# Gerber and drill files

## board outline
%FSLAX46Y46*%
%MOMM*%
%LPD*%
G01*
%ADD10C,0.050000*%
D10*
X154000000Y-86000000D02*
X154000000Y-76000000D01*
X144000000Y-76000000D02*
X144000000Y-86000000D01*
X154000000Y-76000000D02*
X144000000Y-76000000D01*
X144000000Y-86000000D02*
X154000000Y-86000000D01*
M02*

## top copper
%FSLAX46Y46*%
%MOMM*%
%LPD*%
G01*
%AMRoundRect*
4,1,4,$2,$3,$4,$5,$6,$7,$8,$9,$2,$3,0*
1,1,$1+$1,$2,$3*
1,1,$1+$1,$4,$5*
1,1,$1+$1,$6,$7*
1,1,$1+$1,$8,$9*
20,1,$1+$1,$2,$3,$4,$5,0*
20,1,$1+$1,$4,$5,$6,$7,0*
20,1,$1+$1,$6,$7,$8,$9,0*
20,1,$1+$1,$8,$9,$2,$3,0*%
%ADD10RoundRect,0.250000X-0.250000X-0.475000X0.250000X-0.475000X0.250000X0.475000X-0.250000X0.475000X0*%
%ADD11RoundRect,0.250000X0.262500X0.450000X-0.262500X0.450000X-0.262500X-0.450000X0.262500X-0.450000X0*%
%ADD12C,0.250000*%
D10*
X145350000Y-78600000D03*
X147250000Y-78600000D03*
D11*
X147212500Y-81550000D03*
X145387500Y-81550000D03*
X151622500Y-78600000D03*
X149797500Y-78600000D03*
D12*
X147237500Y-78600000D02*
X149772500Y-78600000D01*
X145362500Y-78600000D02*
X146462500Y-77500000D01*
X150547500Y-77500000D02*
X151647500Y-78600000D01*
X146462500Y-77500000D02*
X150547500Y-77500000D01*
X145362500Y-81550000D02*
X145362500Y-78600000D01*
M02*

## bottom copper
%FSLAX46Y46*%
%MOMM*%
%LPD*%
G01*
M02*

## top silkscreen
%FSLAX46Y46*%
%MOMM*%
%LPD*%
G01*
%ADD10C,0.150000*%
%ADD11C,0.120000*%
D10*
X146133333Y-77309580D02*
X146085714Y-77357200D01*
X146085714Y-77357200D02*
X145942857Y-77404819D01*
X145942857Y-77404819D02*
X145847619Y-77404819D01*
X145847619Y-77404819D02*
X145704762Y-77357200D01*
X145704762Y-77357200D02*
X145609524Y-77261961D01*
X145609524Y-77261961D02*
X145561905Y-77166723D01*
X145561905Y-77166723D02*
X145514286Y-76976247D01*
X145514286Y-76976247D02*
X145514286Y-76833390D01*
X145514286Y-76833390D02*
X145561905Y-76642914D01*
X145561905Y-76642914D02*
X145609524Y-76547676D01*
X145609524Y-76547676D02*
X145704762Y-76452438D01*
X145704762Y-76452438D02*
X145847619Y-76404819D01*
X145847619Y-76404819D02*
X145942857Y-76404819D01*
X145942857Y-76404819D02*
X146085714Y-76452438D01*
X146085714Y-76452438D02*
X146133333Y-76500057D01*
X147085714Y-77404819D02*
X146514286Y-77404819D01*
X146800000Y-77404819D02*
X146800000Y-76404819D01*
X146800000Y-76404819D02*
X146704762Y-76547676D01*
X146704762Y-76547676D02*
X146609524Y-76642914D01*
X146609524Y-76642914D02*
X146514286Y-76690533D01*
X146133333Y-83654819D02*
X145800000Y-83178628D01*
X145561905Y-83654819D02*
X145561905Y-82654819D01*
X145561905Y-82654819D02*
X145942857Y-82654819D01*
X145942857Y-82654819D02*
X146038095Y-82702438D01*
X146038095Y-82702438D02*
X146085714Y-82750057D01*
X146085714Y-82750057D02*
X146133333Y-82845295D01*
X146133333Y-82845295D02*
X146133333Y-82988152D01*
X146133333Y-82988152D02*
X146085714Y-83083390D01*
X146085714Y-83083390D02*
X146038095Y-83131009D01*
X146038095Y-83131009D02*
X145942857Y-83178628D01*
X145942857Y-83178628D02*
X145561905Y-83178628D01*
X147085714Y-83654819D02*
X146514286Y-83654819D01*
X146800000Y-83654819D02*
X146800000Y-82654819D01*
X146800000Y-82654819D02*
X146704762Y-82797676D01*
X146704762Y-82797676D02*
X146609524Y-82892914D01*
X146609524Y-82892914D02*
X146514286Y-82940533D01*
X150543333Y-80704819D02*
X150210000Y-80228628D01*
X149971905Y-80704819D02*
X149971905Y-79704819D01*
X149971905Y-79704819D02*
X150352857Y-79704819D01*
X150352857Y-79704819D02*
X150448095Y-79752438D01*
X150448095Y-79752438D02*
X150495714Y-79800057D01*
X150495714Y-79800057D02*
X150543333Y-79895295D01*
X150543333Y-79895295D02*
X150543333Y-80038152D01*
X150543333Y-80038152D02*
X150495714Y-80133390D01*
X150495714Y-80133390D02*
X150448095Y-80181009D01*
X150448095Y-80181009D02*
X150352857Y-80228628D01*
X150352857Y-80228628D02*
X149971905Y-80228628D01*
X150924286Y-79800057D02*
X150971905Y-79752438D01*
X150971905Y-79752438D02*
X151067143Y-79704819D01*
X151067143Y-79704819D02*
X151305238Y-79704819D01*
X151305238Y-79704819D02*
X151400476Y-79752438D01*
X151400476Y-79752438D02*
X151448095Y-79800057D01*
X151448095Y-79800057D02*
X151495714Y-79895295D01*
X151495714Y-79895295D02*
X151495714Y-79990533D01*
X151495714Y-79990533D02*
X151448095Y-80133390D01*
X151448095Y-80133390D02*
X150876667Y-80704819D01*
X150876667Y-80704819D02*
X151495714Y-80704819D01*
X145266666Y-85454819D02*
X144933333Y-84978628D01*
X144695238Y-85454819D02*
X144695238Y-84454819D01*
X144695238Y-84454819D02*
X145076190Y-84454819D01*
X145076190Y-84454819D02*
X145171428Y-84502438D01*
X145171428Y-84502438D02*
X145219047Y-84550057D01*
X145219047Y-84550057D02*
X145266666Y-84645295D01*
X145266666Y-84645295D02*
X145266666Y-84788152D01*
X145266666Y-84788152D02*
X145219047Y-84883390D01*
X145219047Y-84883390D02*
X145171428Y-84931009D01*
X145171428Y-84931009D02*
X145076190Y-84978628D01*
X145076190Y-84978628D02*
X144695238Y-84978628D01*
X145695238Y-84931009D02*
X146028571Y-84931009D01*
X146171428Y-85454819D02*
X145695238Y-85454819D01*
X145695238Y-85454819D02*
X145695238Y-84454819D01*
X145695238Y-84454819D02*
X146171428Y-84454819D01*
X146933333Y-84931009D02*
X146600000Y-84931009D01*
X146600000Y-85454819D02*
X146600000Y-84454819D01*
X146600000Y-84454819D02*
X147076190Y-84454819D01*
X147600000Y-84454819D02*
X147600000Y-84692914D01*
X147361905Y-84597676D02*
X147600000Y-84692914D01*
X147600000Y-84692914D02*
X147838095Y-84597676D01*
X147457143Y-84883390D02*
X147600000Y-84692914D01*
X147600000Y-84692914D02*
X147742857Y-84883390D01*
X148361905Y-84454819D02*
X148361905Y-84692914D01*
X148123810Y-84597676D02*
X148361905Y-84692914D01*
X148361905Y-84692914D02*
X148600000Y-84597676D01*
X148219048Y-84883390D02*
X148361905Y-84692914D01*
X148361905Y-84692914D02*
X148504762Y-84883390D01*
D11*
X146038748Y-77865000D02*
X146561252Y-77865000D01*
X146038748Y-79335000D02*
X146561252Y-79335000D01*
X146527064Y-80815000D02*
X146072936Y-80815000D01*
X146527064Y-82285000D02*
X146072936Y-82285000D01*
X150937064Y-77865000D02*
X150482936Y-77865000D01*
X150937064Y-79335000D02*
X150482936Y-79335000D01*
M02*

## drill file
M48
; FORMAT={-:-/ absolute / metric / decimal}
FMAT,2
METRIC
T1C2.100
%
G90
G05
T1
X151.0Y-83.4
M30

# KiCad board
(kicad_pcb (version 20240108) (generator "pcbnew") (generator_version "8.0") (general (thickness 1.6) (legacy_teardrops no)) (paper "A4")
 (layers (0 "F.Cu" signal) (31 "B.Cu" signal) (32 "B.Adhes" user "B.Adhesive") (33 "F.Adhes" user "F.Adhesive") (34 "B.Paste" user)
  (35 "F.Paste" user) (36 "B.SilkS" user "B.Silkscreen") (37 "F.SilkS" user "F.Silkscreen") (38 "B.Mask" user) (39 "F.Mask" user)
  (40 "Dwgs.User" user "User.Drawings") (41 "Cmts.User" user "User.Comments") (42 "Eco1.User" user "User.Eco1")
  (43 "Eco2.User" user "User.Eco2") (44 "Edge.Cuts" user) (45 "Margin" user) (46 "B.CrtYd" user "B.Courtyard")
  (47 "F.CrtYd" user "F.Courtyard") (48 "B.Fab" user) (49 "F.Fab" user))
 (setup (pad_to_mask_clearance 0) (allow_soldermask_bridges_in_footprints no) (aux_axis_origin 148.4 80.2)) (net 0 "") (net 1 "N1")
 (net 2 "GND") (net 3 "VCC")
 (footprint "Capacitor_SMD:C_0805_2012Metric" (layer "F.Cu") (at 146.3 78.6)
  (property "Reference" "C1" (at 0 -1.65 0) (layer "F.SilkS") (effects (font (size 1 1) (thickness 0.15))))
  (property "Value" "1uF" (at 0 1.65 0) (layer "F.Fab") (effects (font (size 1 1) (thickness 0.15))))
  (fp_line (start -0.261252 -0.735) (end 0.261252 -0.735) (stroke (width 0.12) (type solid)) (layer "F.SilkS"))
  (fp_line (start -0.261252 0.735) (end 0.261252 0.735) (stroke (width 0.12) (type solid)) (layer "F.SilkS"))
  (pad "1" smd roundrect (at -0.95 0) (size 1 1.45) (layers "F.Cu" "F.Paste" "F.Mask") (roundrect_rratio 0.25) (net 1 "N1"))
  (pad "2" smd roundrect (at 0.95 0) (size 1 1.45) (layers "F.Cu" "F.Paste" "F.Mask") (roundrect_rratio 0.25) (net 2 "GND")))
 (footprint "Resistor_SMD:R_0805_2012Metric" (layer "F.Cu") (at 146.3 81.55 180)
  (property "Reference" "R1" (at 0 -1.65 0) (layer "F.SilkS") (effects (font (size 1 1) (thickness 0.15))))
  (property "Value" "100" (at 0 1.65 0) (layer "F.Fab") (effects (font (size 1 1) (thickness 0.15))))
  (fp_line (start -0.227064 0.735) (end 0.227064 0.735) (stroke (width 0.12) (type solid)) (layer "F.SilkS"))
  (fp_line (start -0.227064 -0.735) (end 0.227064 -0.735) (stroke (width 0.12) (type solid)) (layer "F.SilkS"))
  (pad "1" smd roundrect (at -0.9125 0 180) (size 1.025 1.4) (layers "F.Cu" "F.Paste" "F.Mask") (roundrect_rratio 0.243902) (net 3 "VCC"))
  (pad "2" smd roundrect (at 0.9125 0 180) (size 1.025 1.4) (layers "F.Cu" "F.Paste" "F.Mask") (roundrect_rratio 0.243902) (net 1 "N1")))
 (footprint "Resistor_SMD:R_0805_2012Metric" (layer "F.Cu") (at 150.71 78.6 180)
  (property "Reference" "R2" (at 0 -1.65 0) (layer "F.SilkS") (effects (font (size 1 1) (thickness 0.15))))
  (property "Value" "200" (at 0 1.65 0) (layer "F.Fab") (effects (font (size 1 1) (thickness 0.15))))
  (fp_line (start -0.227064 0.735) (end 0.227064 0.735) (stroke (width 0.12) (type solid)) (layer "F.SilkS"))
  (fp_line (start -0.227064 -0.735) (end 0.227064 -0.735) (stroke (width 0.12) (type solid)) (layer "F.SilkS"))
  (pad "1" smd roundrect (at -0.9125 0 180) (size 1.025 1.4) (layers "F.Cu" "F.Paste" "F.Mask") (roundrect_rratio 0.243902) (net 1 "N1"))
  (pad "2" smd roundrect (at 0.9125 0 180) (size 1.025 1.4) (layers "F.Cu" "F.Paste" "F.Mask") (roundrect_rratio 0.243902) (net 2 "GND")))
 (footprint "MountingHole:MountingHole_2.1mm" (layer "F.Cu") (at 151 83.4)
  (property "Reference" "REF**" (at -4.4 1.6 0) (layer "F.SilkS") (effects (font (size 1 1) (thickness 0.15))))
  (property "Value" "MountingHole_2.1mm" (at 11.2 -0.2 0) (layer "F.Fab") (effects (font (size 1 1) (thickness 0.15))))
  (pad "" np_thru_hole circle (at 0 0) (size 2.1 2.1) (drill 2.1) (layers "*.Cu" "*.Mask")))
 (gr_line (start 154 86) (end 154 76) (stroke (width 0.05) (type solid)) (layer "Edge.Cuts"))
 (gr_line (start 144 76) (end 144 86) (stroke (width 0.05) (type solid)) (layer "Edge.Cuts"))
 (gr_line (start 154 76) (end 144 76) (stroke (width 0.05) (type solid)) (layer "Edge.Cuts"))
 (gr_line (start 144 86) (end 154 86) (stroke (width 0.05) (type solid)) (layer "Edge.Cuts"))
 (segment (start 147.2375 78.6) (end 149.7725 78.6) (width 0.25) (layer "F.Cu") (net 2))
 (segment (start 145.3625 78.6) (end 146.4625 77.5) (width 0.25) (layer "F.Cu") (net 1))
 (segment (start 150.5475 77.5) (end 151.6475 78.6) (width 0.25) (layer "F.Cu") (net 1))
 (segment (start 146.4625 77.5) (end 150.5475 77.5) (width 0.25) (layer "F.Cu") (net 1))
 (segment (start 145.3625 81.55) (end 145.3625 78.6) (width 0.25) (layer "F.Cu") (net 1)))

